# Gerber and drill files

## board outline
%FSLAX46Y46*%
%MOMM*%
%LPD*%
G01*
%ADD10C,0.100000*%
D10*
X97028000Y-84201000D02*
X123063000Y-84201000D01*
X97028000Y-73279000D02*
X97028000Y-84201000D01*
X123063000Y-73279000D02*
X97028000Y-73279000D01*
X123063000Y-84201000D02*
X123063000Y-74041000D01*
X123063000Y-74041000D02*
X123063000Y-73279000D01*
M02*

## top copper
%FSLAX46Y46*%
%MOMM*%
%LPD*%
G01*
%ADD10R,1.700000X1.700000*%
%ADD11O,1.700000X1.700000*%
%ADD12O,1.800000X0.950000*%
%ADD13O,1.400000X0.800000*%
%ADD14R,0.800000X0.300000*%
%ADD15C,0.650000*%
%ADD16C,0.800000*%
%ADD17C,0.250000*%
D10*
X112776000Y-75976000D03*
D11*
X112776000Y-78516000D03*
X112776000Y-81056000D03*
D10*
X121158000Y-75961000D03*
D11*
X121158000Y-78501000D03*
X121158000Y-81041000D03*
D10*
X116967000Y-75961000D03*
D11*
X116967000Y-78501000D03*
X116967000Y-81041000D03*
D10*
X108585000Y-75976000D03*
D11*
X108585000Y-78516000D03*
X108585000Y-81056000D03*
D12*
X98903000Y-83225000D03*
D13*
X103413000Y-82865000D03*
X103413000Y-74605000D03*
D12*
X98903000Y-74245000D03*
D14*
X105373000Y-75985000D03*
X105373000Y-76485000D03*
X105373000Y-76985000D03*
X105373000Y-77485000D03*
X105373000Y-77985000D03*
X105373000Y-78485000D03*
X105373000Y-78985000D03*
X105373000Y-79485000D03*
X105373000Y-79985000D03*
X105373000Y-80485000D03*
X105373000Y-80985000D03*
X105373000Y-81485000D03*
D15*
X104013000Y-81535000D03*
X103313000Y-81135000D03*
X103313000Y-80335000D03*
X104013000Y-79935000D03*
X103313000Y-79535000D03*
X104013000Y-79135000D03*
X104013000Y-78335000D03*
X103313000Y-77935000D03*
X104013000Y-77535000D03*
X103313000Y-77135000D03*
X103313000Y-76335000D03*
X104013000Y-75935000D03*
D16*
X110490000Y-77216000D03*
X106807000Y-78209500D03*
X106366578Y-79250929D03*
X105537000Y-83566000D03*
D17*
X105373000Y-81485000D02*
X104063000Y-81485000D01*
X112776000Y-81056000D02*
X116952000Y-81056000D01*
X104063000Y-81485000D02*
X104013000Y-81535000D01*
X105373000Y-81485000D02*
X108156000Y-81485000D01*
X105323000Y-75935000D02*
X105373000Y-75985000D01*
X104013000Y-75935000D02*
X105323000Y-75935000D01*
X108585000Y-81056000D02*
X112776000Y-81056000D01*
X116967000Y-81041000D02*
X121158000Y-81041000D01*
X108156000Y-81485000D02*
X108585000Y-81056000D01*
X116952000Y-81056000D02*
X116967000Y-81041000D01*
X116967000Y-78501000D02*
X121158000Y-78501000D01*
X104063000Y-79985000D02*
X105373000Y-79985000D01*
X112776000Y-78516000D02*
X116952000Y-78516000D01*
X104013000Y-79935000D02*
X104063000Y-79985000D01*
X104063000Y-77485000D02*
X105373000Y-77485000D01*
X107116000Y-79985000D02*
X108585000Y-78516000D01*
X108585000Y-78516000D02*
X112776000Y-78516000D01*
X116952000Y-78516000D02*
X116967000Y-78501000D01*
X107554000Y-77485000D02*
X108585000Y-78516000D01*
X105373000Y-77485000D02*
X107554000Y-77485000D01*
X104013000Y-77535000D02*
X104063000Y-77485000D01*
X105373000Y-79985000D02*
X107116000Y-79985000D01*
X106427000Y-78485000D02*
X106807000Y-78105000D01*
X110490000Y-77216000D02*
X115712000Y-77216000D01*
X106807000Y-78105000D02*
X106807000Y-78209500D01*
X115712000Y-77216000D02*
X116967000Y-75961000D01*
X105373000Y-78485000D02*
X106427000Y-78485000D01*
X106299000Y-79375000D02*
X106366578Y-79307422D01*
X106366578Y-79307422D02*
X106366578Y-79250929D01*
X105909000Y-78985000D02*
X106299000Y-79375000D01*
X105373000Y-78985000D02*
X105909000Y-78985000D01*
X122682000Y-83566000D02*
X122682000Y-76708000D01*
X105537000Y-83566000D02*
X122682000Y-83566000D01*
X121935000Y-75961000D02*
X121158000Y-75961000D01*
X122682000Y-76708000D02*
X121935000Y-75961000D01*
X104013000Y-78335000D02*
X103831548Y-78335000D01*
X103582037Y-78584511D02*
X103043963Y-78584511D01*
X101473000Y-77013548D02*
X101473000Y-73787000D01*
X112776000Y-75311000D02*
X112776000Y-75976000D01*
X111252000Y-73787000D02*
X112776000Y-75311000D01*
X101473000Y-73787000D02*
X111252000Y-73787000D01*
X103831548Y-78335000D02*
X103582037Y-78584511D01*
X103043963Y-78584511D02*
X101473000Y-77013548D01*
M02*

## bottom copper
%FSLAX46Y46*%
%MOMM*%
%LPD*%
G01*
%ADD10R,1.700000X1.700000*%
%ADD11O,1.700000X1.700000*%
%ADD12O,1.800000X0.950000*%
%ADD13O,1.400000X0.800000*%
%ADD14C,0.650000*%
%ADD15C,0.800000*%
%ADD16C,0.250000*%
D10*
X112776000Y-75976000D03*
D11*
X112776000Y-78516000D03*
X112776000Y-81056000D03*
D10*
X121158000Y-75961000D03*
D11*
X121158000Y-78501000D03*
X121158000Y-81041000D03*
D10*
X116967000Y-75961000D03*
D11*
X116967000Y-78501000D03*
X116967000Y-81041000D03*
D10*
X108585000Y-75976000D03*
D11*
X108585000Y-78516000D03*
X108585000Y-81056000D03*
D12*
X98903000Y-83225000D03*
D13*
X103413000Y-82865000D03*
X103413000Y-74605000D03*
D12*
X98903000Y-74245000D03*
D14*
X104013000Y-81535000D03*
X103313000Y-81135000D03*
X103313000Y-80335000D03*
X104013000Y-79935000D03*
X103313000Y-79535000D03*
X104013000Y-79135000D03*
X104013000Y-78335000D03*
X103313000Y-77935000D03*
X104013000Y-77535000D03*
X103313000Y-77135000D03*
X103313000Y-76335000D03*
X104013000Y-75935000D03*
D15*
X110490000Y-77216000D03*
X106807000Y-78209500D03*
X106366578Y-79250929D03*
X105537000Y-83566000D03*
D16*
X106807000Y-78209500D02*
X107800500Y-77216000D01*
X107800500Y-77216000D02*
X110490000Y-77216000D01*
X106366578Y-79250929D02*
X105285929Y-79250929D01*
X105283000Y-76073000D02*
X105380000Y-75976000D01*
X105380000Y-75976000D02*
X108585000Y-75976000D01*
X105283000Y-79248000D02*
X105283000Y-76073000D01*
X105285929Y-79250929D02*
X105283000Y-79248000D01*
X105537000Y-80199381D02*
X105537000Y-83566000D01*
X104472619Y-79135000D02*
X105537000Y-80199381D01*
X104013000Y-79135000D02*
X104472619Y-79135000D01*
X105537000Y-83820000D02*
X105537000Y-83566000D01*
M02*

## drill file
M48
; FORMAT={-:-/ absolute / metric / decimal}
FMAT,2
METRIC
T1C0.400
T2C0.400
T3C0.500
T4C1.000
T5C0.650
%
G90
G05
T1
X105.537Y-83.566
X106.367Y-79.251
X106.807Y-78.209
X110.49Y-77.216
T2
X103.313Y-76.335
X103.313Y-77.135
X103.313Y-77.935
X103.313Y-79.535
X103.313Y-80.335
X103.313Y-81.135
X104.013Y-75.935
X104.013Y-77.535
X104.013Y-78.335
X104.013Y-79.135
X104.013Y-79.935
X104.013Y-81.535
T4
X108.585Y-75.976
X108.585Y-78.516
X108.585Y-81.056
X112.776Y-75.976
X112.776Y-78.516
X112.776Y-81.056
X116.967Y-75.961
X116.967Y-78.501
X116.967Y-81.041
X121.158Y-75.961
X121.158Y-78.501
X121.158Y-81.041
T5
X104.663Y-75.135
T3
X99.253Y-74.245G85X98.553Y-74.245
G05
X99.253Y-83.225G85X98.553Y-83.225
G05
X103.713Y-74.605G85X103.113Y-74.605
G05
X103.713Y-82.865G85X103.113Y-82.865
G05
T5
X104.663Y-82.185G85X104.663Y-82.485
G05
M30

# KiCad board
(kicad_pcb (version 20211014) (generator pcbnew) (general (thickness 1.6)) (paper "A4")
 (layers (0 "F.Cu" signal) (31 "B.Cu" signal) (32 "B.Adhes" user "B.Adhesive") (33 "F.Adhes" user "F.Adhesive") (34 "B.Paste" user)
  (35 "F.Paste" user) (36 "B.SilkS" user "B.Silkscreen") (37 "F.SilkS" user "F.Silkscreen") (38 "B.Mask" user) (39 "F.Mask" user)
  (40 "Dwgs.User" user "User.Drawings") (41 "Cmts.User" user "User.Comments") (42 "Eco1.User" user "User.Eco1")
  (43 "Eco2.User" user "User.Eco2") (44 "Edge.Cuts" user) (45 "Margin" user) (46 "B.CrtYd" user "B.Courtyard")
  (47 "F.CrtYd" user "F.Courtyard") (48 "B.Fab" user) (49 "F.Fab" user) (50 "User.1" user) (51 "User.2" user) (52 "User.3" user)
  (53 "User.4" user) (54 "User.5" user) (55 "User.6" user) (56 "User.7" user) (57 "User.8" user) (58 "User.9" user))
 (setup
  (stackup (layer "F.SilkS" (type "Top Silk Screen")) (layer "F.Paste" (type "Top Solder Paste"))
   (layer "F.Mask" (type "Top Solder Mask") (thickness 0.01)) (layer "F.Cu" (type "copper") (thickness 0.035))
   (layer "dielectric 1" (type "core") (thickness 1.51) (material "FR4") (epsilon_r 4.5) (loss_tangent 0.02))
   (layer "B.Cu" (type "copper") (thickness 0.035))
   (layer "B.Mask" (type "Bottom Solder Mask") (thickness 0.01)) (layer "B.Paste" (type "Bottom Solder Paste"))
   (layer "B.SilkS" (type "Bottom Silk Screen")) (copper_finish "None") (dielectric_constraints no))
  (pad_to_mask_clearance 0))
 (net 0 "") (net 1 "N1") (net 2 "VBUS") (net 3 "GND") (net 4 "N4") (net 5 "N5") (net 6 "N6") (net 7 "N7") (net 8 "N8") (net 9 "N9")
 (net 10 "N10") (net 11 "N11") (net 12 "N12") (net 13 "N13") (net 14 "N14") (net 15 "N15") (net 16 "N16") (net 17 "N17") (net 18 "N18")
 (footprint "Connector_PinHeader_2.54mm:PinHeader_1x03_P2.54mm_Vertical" (layer "F.Cu") (at 112.776 75.976)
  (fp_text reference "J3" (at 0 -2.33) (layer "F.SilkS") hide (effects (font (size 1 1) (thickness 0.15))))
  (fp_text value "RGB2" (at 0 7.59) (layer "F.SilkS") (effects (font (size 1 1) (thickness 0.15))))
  (pad "1" thru_hole rect (at 0 0) (size 1.7 1.7) (drill 1) (layers *.Cu *.Mask) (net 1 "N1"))
  (pad "2" thru_hole oval (at 0 2.54) (size 1.7 1.7) (drill 1) (layers *.Cu *.Mask) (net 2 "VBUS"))
  (pad "3" thru_hole oval (at 0 5.08) (size 1.7 1.7) (drill 1) (layers *.Cu *.Mask) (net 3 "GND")))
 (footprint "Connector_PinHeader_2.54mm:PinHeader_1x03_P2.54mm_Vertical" (layer "F.Cu") (at 121.158 75.961)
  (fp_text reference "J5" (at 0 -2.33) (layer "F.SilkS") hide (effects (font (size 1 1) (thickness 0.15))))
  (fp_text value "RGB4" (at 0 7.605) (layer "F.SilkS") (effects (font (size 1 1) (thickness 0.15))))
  (pad "1" thru_hole rect (at 0 0) (size 1.7 1.7) (drill 1) (layers *.Cu *.Mask) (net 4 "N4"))
  (pad "2" thru_hole oval (at 0 2.54) (size 1.7 1.7) (drill 1) (layers *.Cu *.Mask) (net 2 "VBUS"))
  (pad "3" thru_hole oval (at 0 5.08) (size 1.7 1.7) (drill 1) (layers *.Cu *.Mask) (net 3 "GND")))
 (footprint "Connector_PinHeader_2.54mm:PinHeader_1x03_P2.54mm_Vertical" (layer "F.Cu") (at 116.967 75.961)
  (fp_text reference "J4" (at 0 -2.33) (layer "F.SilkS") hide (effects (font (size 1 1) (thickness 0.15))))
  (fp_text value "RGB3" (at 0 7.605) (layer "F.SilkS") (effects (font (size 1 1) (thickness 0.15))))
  (pad "1" thru_hole rect (at 0 0) (size 1.7 1.7) (drill 1) (layers *.Cu *.Mask) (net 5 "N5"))
  (pad "2" thru_hole oval (at 0 2.54) (size 1.7 1.7) (drill 1) (layers *.Cu *.Mask) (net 2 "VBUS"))
  (pad "3" thru_hole oval (at 0 5.08) (size 1.7 1.7) (drill 1) (layers *.Cu *.Mask) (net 3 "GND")))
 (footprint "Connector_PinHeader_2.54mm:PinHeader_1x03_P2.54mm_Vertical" (layer "F.Cu") (at 108.585 75.976)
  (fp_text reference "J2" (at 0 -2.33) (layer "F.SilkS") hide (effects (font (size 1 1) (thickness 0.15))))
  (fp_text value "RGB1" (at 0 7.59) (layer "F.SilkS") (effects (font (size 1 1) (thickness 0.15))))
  (pad "1" thru_hole rect (at 0 0) (size 1.7 1.7) (drill 1) (layers *.Cu *.Mask) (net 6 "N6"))
  (pad "2" thru_hole oval (at 0 2.54) (size 1.7 1.7) (drill 1) (layers *.Cu *.Mask) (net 2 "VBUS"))
  (pad "3" thru_hole oval (at 0 5.08) (size 1.7 1.7) (drill 1) (layers *.Cu *.Mask) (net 3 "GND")))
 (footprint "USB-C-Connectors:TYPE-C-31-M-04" (layer "F.Cu") (at 100.303 78.735 -90)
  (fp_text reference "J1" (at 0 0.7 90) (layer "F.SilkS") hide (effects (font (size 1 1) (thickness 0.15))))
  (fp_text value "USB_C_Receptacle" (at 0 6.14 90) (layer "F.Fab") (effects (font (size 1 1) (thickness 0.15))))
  (pad "" np_thru_hole circle locked (at -3.6 -4.36 270) (size 0.65 0.65) (drill 0.65) (layers *.Cu *.Mask))
  (pad "" np_thru_hole oval locked (at 3.6 -4.36 270) (size 0.95 0.65) (drill oval 0.95 0.65) (layers *.Cu *.Mask))
  (pad "31" thru_hole oval locked (at 4.49 1.4 270) (size 0.95 1.8) (drill oval 0.5 1.2) (layers *.Cu *.Mask))
  (pad "32" thru_hole oval locked (at 4.13 -3.11 270) (size 0.8 1.4) (drill oval 0.5 1.1) (layers *.Cu *.Mask))
  (pad "33" thru_hole oval locked (at -4.13 -3.11 270) (size 0.8 1.4) (drill oval 0.5 1.1) (layers *.Cu *.Mask))
  (pad "34" thru_hole oval locked (at -4.49 1.4 270) (size 0.95 1.8) (drill oval 0.5 1.2) (layers *.Cu *.Mask))
  (pad "A1" smd rect locked (at -2.75 -5.07 270) (size 0.3 0.8) (layers "F.Cu" "F.Paste" "F.Mask") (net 3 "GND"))
  (pad "A2" smd rect locked (at -2.25 -5.07 270) (size 0.3 0.8) (layers "F.Cu" "F.Paste" "F.Mask") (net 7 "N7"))
  (pad "A3" smd rect locked (at -1.75 -5.07 270) (size 0.3 0.8) (layers "F.Cu" "F.Paste" "F.Mask") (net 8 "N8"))
  (pad "A4" smd rect locked (at -1.25 -5.07 270) (size 0.3 0.8) (layers "F.Cu" "F.Paste" "F.Mask") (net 2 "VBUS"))
  (pad "A5" smd rect locked (at -0.75 -5.07 270) (size 0.3 0.8) (layers "F.Cu" "F.Paste" "F.Mask") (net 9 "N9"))
  (pad "A6" smd rect locked (at -0.25 -5.07 270) (size 0.3 0.8) (layers "F.Cu" "F.Paste" "F.Mask") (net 5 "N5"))
  (pad "A7" smd rect locked (at 0.25 -5.07 270) (size 0.3 0.8) (layers "F.Cu" "F.Paste" "F.Mask") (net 6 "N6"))
  (pad "A8" smd rect locked (at 0.75 -5.07 270) (size 0.3 0.8) (layers "F.Cu" "F.Paste" "F.Mask") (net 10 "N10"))
  (pad "A9" smd rect locked (at 1.25 -5.07 270) (size 0.3 0.8) (layers "F.Cu" "F.Paste" "F.Mask") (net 2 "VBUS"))
  (pad "A10" smd rect locked (at 1.75 -5.07 270) (size 0.3 0.8) (layers "F.Cu" "F.Paste" "F.Mask") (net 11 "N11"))
  (pad "A11" smd rect locked (at 2.25 -5.07 270) (size 0.3 0.8) (layers "F.Cu" "F.Paste" "F.Mask") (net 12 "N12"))
  (pad "A12" smd rect locked (at 2.75 -5.07 270) (size 0.3 0.8) (layers "F.Cu" "F.Paste" "F.Mask") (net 3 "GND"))
  (pad "B1" thru_hole circle locked (at 2.8 -3.71 270) (size 0.65 0.65) (drill 0.4) (layers *.Cu *.Mask) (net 3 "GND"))
  (pad "B2" thru_hole circle locked (at 2.4 -3.01 270) (size 0.65 0.65) (drill 0.4) (layers *.Cu *.Mask) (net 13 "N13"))
  (pad "B3" thru_hole circle locked (at 1.6 -3.01 270) (size 0.65 0.65) (drill 0.4) (layers *.Cu *.Mask) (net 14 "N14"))
  (pad "B4" thru_hole circle locked (at 1.2 -3.71 270) (size 0.65 0.65) (drill 0.4) (layers *.Cu *.Mask) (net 2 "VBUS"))
  (pad "B5" thru_hole circle locked (at 0.8 -3.01 270) (size 0.65 0.65) (drill 0.4) (layers *.Cu *.Mask) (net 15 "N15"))
  (pad "B6" thru_hole circle locked (at 0.4 -3.71 270) (size 0.65 0.65) (drill 0.4) (layers *.Cu *.Mask) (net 4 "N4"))
  (pad "B7" thru_hole circle locked (at -0.4 -3.71 270) (size 0.65 0.65) (drill 0.4) (layers *.Cu *.Mask) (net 1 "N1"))
  (pad "B8" thru_hole circle locked (at -0.8 -3.01 270) (size 0.65 0.65) (drill 0.4) (layers *.Cu *.Mask) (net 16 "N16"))
  (pad "B9" thru_hole circle locked (at -1.2 -3.71 270) (size 0.65 0.65) (drill 0.4) (layers *.Cu *.Mask) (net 2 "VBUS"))
  (pad "B10" thru_hole circle locked (at -1.6 -3.01 270) (size 0.65 0.65) (drill 0.4) (layers *.Cu *.Mask) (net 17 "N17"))
  (pad "B11" thru_hole circle locked (at -2.4 -3.01 270) (size 0.65 0.65) (drill 0.4) (layers *.Cu *.Mask) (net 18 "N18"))
  (pad "B12" thru_hole circle locked (at -2.8 -3.71 270) (size 0.65 0.65) (drill 0.4) (layers *.Cu *.Mask) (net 3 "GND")))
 (gr_line (start 97.028 84.201) (end 123.063 84.201) (layer "Edge.Cuts") (width 0.1))
 (gr_line (start 97.028 73.279) (end 97.028 84.201) (layer "Edge.Cuts") (width 0.1))
 (gr_line (start 123.063 73.279) (end 97.028 73.279) (layer "Edge.Cuts") (width 0.1))
 (gr_line (start 123.063 84.201) (end 123.063 74.041) (layer "Edge.Cuts") (width 0.1))
 (gr_line (start 123.063 74.041) (end 123.063 73.279) (layer "Edge.Cuts") (width 0.1))
 (segment (start 105.373 81.485) (end 104.063 81.485) (width 0.25) (layer "F.Cu") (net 3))
 (segment (start 112.776 81.056) (end 116.952 81.056) (width 0.25) (layer "F.Cu") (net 3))
 (segment (start 104.063 81.485) (end 104.013 81.535) (width 0.25) (layer "F.Cu") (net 3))
 (segment (start 105.373 81.485) (end 108.156 81.485) (width 0.25) (layer "F.Cu") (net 3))
 (segment (start 105.323 75.935) (end 105.373 75.985) (width 0.25) (layer "F.Cu") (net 3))
 (segment (start 104.013 75.935) (end 105.323 75.935) (width 0.25) (layer "F.Cu") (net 3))
 (segment (start 108.585 81.056) (end 112.776 81.056) (width 0.25) (layer "F.Cu") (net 3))
 (segment (start 116.967 81.041) (end 121.158 81.041) (width 0.25) (layer "F.Cu") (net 3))
 (segment (start 108.156 81.485) (end 108.585 81.056) (width 0.25) (layer "F.Cu") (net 3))
 (segment (start 116.952 81.056) (end 116.967 81.041) (width 0.25) (layer "F.Cu") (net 3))
 (segment (start 116.967 78.501) (end 121.158 78.501) (width 0.25) (layer "F.Cu") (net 2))
 (segment (start 104.063 79.985) (end 105.373 79.985) (width 0.25) (layer "F.Cu") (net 2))
 (segment (start 112.776 78.516) (end 116.952 78.516) (width 0.25) (layer "F.Cu") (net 2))
 (segment (start 104.013 79.935) (end 104.063 79.985) (width 0.25) (layer "F.Cu") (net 2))
 (segment (start 104.063 77.485) (end 105.373 77.485) (width 0.25) (layer "F.Cu") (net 2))
 (segment (start 107.116 79.985) (end 108.585 78.516) (width 0.25) (layer "F.Cu") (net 2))
 (segment (start 108.585 78.516) (end 112.776 78.516) (width 0.25) (layer "F.Cu") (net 2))
 (segment (start 116.952 78.516) (end 116.967 78.501) (width 0.25) (layer "F.Cu") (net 2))
 (segment (start 107.554 77.485) (end 108.585 78.516) (width 0.25) (layer "F.Cu") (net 2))
 (segment (start 105.373 77.485) (end 107.554 77.485) (width 0.25) (layer "F.Cu") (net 2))
 (segment (start 104.013 77.535) (end 104.063 77.485) (width 0.25) (layer "F.Cu") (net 2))
 (segment (start 105.373 79.985) (end 107.116 79.985) (width 0.25) (layer "F.Cu") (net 2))
 (segment (start 106.427 78.485) (end 106.807 78.105) (width 0.25) (layer "F.Cu") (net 5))
 (segment (start 110.49 77.216) (end 115.712 77.216) (width 0.25) (layer "F.Cu") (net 5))
 (segment (start 106.807 78.105) (end 106.807 78.2095) (width 0.25) (layer "F.Cu") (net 5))
 (segment (start 115.712 77.216) (end 116.967 75.961) (width 0.25) (layer "F.Cu") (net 5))
 (segment (start 105.373 78.485) (end 106.427 78.485) (width 0.25) (layer "F.Cu") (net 5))
 (via (at 110.49 77.216) (size 0.8) (drill 0.4) (layers "F.Cu" "B.Cu") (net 5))
 (via (at 106.807 78.2095) (size 0.8) (drill 0.4) (layers "F.Cu" "B.Cu") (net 5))
 (segment (start 106.807 78.2095) (end 107.8005 77.216) (width 0.25) (layer "B.Cu") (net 5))
 (segment (start 107.8005 77.216) (end 110.49 77.216) (width 0.25) (layer "B.Cu") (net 5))
 (segment (start 106.299 79.375) (end 106.366578 79.307422) (width 0.25) (layer "F.Cu") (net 6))
 (segment (start 106.366578 79.307422) (end 106.366578 79.250929) (width 0.25) (layer "F.Cu") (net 6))
 (segment (start 105.909 78.985) (end 106.299 79.375) (width 0.25) (layer "F.Cu") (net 6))
 (segment (start 105.373 78.985) (end 105.909 78.985) (width 0.25) (layer "F.Cu") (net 6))
 (via (at 106.366578 79.250929) (size 0.8) (drill 0.4) (layers "F.Cu" "B.Cu") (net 6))
 (segment (start 106.366578 79.250929) (end 105.285929 79.250929) (width 0.25) (layer "B.Cu") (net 6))
 (segment (start 105.283 76.073) (end 105.38 75.976) (width 0.25) (layer "B.Cu") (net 6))
 (segment (start 105.38 75.976) (end 108.585 75.976) (width 0.25) (layer "B.Cu") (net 6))
 (segment (start 105.283 79.248) (end 105.283 76.073) (width 0.25) (layer "B.Cu") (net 6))
 (segment (start 105.285929 79.250929) (end 105.283 79.248) (width 0.25) (layer "B.Cu") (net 6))
 (segment (start 122.682 83.566) (end 122.682 76.708) (width 0.25) (layer "F.Cu") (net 4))
 (segment (start 105.537 83.566) (end 122.682 83.566) (width 0.25) (layer "F.Cu") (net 4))
 (segment (start 121.935 75.961) (end 121.158 75.961) (width 0.25) (layer "F.Cu") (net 4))
 (segment (start 122.682 76.708) (end 121.935 75.961) (width 0.25) (layer "F.Cu") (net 4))
 (via (at 105.537 83.566) (size 0.8) (drill 0.4) (layers "F.Cu" "B.Cu") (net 4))
 (segment (start 105.537 80.199381) (end 105.537 83.566) (width 0.25) (layer "B.Cu") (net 4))
 (segment (start 104.472619 79.135) (end 105.537 80.199381) (width 0.25) (layer "B.Cu") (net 4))
 (segment (start 104.013 79.135) (end 104.472619 79.135) (width 0.25) (layer "B.Cu") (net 4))
 (segment (start 105.537 83.82) (end 105.537 83.566) (width 0.25) (layer "B.Cu") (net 4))
 (segment (start 104.013 78.335) (end 103.831548 78.335) (width 0.25) (layer "F.Cu") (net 1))
 (segment (start 103.582037 78.584511) (end 103.043963 78.584511) (width 0.25) (layer "F.Cu") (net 1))
 (segment (start 101.473 77.013548) (end 101.473 73.787) (width 0.25) (layer "F.Cu") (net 1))
 (segment (start 112.776 75.311) (end 112.776 75.976) (width 0.25) (layer "F.Cu") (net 1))
 (segment (start 111.252 73.787) (end 112.776 75.311) (width 0.25) (layer "F.Cu") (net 1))
 (segment (start 101.473 73.787) (end 111.252 73.787) (width 0.25) (layer "F.Cu") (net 1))
 (segment (start 103.831548 78.335) (end 103.582037 78.584511) (width 0.25) (layer "F.Cu") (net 1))
 (segment (start 103.043963 78.584511) (end 101.473 77.013548) (width 0.25) (layer "F.Cu") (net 1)))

